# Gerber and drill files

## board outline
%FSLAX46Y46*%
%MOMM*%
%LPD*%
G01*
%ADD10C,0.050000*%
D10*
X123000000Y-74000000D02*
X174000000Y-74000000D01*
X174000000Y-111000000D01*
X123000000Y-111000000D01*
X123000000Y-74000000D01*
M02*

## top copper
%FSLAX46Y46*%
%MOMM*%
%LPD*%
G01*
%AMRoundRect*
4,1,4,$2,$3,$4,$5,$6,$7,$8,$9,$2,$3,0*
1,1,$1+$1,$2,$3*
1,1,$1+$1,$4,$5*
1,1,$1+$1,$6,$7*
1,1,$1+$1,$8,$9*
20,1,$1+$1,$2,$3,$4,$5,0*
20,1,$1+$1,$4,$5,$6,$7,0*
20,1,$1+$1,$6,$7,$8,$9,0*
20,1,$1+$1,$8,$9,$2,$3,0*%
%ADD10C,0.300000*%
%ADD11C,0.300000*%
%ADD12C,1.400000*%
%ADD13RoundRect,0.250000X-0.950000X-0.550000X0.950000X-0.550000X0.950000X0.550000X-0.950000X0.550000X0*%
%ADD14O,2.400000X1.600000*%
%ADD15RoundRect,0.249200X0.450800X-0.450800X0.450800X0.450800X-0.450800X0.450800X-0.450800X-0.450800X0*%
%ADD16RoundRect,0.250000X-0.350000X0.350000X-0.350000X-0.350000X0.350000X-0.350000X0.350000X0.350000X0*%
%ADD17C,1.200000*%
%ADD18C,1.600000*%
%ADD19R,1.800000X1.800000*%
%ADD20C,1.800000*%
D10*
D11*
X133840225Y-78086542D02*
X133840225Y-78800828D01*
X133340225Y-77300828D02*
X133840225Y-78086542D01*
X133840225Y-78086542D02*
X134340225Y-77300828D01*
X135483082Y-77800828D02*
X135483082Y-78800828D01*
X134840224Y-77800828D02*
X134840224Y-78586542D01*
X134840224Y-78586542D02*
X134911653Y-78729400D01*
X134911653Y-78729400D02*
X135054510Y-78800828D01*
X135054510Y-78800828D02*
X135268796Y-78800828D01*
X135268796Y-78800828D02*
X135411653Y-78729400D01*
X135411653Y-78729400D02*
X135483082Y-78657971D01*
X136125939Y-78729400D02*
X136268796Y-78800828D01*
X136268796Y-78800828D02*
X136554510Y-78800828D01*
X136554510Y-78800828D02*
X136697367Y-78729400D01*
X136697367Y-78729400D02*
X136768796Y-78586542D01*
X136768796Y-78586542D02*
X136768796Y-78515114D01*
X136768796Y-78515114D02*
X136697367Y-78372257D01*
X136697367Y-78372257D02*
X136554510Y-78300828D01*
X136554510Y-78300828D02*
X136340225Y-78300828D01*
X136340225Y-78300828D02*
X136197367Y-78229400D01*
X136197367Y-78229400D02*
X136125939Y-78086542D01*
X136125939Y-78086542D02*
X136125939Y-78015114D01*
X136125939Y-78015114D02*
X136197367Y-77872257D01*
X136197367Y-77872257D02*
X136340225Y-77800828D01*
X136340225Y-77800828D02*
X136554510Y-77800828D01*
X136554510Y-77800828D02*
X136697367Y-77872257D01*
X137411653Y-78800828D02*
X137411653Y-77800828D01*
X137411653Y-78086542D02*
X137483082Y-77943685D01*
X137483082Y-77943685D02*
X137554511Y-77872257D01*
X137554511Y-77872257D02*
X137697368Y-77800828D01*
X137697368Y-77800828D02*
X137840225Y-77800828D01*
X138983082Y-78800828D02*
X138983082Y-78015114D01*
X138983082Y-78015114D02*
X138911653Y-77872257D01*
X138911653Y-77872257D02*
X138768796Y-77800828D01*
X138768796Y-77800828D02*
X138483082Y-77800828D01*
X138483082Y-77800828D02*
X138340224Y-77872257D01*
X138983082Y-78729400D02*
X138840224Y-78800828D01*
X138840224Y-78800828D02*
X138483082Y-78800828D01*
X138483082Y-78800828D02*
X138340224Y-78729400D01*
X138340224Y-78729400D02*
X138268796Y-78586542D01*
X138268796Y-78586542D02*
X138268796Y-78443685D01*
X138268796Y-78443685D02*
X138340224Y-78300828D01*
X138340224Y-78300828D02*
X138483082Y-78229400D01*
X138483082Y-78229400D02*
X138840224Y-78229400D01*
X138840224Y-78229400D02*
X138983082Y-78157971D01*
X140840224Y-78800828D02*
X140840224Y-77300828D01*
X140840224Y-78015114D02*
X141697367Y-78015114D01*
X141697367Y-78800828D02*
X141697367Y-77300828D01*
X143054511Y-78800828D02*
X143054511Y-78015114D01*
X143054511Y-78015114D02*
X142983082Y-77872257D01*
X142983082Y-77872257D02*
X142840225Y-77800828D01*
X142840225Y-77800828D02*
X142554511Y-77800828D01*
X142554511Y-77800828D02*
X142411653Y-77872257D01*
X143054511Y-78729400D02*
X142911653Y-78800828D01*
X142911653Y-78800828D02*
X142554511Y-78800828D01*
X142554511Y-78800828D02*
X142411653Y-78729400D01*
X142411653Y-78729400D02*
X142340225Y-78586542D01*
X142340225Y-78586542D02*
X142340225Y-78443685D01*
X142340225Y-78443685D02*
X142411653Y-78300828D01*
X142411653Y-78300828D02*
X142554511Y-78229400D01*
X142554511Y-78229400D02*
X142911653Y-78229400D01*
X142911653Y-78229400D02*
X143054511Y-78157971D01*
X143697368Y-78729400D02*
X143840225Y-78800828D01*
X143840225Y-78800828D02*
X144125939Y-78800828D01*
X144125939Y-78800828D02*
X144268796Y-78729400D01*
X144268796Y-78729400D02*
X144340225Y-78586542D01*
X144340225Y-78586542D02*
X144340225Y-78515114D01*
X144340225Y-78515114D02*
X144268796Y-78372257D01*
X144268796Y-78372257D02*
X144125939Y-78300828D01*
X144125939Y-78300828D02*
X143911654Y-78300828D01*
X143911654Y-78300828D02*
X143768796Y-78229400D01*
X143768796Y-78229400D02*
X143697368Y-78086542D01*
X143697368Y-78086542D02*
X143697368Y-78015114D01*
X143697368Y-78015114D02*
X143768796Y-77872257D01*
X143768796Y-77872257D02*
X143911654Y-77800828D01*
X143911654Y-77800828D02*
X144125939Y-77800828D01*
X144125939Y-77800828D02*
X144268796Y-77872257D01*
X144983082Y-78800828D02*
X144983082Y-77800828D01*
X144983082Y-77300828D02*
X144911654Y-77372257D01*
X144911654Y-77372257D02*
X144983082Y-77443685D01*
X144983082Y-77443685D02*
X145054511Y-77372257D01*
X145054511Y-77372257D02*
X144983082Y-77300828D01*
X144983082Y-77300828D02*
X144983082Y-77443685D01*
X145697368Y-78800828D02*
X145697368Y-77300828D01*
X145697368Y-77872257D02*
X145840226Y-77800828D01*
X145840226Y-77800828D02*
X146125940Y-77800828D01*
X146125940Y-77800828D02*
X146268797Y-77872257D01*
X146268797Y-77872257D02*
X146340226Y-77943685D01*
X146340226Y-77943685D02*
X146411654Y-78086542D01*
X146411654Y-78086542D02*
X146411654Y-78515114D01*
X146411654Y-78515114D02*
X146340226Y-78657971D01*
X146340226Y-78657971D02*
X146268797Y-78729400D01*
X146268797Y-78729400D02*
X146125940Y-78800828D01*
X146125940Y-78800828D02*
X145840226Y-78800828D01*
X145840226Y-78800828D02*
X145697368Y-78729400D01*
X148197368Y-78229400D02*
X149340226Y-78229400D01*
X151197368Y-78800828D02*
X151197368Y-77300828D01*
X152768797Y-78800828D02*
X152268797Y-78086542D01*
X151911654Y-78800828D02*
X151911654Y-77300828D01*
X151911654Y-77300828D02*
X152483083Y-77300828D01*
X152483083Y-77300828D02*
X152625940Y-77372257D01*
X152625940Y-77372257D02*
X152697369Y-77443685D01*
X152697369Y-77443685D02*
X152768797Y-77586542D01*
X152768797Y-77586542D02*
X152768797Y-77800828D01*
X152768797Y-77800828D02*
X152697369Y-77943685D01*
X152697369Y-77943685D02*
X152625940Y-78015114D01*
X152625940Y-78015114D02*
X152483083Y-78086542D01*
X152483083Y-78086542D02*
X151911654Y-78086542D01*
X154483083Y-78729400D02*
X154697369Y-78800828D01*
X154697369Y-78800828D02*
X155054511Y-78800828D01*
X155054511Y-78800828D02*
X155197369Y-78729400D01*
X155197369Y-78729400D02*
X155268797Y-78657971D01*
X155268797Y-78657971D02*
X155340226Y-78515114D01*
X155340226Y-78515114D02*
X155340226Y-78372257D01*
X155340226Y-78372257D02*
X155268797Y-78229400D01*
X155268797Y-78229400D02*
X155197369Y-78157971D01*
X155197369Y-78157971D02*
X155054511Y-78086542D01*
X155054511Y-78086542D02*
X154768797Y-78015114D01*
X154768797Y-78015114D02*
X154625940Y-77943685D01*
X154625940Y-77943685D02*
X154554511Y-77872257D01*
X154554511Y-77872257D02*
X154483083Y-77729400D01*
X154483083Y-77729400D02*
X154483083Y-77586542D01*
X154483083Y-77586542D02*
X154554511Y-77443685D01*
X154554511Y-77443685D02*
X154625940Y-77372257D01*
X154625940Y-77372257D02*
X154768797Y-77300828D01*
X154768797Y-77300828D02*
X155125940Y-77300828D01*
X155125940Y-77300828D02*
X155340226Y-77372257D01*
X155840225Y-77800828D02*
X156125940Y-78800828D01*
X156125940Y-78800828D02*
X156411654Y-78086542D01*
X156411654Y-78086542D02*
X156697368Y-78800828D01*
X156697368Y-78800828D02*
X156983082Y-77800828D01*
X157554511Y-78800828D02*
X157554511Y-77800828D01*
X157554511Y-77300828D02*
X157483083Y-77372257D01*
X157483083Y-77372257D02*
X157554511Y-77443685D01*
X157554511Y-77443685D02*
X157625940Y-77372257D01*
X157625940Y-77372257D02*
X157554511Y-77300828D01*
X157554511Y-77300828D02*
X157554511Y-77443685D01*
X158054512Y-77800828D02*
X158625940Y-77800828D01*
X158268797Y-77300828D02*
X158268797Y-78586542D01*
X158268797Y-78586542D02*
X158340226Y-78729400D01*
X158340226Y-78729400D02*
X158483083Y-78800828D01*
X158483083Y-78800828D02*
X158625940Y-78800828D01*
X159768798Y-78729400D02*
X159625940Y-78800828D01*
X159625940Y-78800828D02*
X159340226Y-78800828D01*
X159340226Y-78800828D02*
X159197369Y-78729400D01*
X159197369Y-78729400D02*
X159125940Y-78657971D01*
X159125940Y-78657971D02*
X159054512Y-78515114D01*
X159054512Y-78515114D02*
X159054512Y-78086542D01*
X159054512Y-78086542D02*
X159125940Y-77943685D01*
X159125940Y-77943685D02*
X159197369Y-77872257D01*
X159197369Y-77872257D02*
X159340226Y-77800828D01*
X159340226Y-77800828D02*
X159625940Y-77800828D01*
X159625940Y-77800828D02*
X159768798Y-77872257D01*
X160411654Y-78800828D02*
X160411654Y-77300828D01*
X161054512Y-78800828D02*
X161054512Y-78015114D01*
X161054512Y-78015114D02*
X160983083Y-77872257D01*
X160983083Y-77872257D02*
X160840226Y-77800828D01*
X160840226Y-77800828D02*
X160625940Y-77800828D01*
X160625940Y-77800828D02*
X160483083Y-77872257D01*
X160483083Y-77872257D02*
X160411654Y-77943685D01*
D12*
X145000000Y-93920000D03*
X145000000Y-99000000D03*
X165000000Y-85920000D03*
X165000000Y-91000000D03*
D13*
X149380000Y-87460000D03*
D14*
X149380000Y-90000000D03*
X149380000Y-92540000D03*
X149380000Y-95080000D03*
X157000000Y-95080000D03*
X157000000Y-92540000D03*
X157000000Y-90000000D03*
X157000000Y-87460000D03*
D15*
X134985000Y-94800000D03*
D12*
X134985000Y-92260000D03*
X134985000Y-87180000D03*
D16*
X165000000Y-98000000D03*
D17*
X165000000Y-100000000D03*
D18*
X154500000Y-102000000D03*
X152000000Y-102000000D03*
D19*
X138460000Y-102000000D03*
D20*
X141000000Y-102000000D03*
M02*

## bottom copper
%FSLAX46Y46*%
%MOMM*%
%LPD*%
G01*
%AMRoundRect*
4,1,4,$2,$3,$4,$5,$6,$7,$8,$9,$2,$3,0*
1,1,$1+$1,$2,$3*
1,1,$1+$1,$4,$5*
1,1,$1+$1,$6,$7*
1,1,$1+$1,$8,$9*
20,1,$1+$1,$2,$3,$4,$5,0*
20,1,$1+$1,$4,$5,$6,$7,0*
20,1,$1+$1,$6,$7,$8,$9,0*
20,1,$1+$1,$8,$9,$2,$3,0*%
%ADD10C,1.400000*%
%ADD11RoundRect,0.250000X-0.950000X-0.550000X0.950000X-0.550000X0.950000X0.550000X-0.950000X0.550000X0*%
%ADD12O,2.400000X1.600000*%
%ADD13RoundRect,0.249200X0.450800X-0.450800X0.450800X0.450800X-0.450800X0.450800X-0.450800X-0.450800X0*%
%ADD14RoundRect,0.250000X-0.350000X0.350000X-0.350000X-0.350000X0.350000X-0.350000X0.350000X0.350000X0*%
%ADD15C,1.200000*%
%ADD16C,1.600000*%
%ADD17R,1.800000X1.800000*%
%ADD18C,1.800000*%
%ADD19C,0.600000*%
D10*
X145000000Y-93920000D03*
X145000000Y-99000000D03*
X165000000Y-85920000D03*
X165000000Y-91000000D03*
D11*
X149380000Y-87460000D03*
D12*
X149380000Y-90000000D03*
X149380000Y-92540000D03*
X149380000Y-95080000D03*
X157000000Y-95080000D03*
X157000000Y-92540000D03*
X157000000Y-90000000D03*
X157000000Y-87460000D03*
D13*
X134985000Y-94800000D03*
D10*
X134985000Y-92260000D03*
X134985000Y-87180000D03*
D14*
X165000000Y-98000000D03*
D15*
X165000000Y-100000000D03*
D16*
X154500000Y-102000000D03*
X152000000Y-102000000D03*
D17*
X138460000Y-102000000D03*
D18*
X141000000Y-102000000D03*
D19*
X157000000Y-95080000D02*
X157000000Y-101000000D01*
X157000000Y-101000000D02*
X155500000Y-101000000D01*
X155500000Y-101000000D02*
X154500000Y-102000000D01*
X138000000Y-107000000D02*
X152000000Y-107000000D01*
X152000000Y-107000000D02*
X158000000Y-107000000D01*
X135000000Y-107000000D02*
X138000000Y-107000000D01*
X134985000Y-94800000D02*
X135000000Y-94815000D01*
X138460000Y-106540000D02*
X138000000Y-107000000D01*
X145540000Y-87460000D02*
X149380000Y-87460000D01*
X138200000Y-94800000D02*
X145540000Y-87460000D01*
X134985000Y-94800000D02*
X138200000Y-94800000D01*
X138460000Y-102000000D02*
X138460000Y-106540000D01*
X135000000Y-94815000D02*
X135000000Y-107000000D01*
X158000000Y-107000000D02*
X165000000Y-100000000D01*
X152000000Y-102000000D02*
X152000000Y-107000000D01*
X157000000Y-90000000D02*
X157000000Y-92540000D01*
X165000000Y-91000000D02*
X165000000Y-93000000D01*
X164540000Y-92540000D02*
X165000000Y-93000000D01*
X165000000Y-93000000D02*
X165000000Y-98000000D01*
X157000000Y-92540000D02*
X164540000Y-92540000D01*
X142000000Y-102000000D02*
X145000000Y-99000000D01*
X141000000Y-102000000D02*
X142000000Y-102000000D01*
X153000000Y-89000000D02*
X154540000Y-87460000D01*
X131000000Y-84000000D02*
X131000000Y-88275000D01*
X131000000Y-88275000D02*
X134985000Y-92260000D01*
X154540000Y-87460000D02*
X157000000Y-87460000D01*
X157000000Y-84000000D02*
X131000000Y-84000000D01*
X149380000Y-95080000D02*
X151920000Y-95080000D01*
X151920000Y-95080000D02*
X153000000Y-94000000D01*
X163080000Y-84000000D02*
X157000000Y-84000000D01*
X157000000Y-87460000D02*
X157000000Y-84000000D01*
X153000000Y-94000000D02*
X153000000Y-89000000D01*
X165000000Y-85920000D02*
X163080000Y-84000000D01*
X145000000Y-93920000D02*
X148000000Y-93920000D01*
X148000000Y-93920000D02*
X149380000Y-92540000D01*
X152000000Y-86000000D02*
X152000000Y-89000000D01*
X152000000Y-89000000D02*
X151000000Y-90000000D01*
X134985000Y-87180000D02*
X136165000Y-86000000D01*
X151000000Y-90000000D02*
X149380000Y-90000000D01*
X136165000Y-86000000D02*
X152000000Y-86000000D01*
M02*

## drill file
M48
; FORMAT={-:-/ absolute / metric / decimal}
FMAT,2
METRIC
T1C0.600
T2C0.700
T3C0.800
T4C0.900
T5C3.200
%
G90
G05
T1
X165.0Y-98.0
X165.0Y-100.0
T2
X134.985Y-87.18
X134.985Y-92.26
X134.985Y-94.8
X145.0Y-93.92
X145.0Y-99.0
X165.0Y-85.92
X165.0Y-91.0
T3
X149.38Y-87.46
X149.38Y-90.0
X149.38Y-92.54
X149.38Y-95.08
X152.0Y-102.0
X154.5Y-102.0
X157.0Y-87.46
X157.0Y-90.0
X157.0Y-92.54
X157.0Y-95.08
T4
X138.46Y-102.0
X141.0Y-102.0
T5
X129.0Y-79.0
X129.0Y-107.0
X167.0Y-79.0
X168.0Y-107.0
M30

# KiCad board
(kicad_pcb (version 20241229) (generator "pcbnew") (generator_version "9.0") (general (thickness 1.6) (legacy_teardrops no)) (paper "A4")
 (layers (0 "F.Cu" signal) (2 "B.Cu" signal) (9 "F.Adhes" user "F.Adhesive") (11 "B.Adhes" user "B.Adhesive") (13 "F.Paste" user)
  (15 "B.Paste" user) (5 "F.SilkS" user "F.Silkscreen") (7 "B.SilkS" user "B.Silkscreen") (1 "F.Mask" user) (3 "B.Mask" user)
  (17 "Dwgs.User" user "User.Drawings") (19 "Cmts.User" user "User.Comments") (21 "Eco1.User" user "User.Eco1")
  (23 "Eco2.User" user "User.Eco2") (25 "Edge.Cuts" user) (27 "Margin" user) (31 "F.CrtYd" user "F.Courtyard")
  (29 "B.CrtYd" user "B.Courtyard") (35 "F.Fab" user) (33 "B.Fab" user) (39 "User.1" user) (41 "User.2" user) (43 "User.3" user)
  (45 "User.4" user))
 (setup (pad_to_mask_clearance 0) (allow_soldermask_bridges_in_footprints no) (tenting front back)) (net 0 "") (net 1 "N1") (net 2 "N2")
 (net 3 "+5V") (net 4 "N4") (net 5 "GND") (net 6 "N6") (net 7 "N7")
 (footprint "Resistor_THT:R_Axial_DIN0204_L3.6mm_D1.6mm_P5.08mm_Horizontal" (layer "F.Cu") (at 145 93.92 -90)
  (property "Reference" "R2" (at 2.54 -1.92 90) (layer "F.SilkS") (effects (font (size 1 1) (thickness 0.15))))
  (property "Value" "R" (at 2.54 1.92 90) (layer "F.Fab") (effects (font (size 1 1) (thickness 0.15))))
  (pad "1" thru_hole circle (at 0 0 270) (size 1.4 1.4) (drill 0.7) (layers "*.Cu" "*.Mask") (remove_unused_layers no) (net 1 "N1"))
  (pad "2" thru_hole circle (at 5.08 0 270) (size 1.4 1.4) (drill 0.7) (layers "*.Cu" "*.Mask") (remove_unused_layers no) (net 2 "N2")))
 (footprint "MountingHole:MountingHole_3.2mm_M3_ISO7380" (layer "F.Cu") (at 168 107)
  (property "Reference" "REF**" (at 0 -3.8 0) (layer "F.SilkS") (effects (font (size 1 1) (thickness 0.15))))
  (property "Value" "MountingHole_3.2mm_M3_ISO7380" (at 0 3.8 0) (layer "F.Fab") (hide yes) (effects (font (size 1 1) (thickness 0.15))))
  (pad "" np_thru_hole circle (at 0 0) (size 3.2 3.2) (drill 3.2) (layers "*.Cu" "*.Mask")))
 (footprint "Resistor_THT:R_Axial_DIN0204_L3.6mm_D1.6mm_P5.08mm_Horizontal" (layer "F.Cu") (at 165 85.92 -90)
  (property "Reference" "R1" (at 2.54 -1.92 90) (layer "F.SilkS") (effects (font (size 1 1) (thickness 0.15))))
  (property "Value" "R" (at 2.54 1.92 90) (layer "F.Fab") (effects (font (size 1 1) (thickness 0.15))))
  (pad "1" thru_hole circle (at 0 0 270) (size 1.4 1.4) (drill 0.7) (layers "*.Cu" "*.Mask") (remove_unused_layers no) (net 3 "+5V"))
  (pad "2" thru_hole circle (at 5.08 0 270) (size 1.4 1.4) (drill 0.7) (layers "*.Cu" "*.Mask") (remove_unused_layers no) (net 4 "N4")))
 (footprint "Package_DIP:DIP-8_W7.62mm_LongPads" (layer "F.Cu") (at 149.38 87.46)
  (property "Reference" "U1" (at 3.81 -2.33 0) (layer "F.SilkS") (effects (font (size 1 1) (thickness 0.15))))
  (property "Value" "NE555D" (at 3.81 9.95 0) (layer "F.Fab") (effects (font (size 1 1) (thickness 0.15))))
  (pad "1" thru_hole roundrect (at 0 0) (size 2.4 1.6) (drill 0.8) (layers "*.Cu" "*.Mask") (remove_unused_layers no)
   (roundrect_rratio 0.15625) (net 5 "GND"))
  (pad "2" thru_hole oval (at 0 2.54) (size 2.4 1.6) (drill 0.8) (layers "*.Cu" "*.Mask") (remove_unused_layers no) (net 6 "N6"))
  (pad "3" thru_hole oval (at 0 5.08) (size 2.4 1.6) (drill 0.8) (layers "*.Cu" "*.Mask") (remove_unused_layers no) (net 1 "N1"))
  (pad "4" thru_hole oval (at 0 7.62) (size 2.4 1.6) (drill 0.8) (layers "*.Cu" "*.Mask") (remove_unused_layers no) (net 3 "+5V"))
  (pad "5" thru_hole oval (at 7.62 7.62) (size 2.4 1.6) (drill 0.8) (layers "*.Cu" "*.Mask") (remove_unused_layers no) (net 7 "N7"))
  (pad "6" thru_hole oval (at 7.62 5.08) (size 2.4 1.6) (drill 0.8) (layers "*.Cu" "*.Mask") (remove_unused_layers no) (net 4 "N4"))
  (pad "7" thru_hole oval (at 7.62 2.54) (size 2.4 1.6) (drill 0.8) (layers "*.Cu" "*.Mask") (remove_unused_layers no) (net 4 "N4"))
  (pad "8" thru_hole oval (at 7.62 0) (size 2.4 1.6) (drill 0.8) (layers "*.Cu" "*.Mask") (remove_unused_layers no) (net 3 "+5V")))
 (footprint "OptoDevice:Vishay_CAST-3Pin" (layer "F.Cu") (at 134.985 94.8 90)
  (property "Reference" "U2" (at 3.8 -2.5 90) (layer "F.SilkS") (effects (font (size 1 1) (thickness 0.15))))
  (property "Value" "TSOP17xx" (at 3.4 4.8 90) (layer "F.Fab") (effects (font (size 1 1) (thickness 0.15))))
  (pad "1" thru_hole roundrect (at 0 0 90) (size 1.4 1.4) (drill 0.7) (layers "*.Cu" "*.Mask") (remove_unused_layers no)
   (roundrect_rratio 0.178) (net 5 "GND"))
  (pad "2" thru_hole circle (at 2.54 0 90) (size 1.4 1.4) (drill 0.7) (layers "*.Cu" "*.Mask") (remove_unused_layers no) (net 3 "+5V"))
  (pad "3" thru_hole circle (at 7.62 0 90) (size 1.4 1.4) (drill 0.7) (layers "*.Cu" "*.Mask") (remove_unused_layers no) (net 6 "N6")))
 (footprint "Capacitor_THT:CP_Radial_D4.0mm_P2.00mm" (layer "F.Cu") (at 165 98 -90)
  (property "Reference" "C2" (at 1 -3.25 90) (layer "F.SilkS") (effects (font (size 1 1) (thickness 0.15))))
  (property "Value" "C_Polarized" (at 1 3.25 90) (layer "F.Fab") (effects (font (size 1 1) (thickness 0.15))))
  (pad "1" thru_hole roundrect (at 0 0 270) (size 1.2 1.2) (drill 0.6) (layers "*.Cu" "*.Mask") (remove_unused_layers no)
   (roundrect_rratio 0.208333) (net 4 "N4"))
  (pad "2" thru_hole circle (at 2 0 270) (size 1.2 1.2) (drill 0.6) (layers "*.Cu" "*.Mask") (remove_unused_layers no) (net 5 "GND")))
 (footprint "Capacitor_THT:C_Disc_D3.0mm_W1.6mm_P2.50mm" (layer "F.Cu") (at 154.5 102 180)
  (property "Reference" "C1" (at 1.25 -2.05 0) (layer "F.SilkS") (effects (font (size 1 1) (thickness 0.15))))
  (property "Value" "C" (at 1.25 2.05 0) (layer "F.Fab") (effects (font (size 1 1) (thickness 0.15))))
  (pad "1" thru_hole circle (at 0 0 180) (size 1.6 1.6) (drill 0.8) (layers "*.Cu" "*.Mask") (remove_unused_layers no) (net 7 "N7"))
  (pad "2" thru_hole circle (at 2.5 0 180) (size 1.6 1.6) (drill 0.8) (layers "*.Cu" "*.Mask") (remove_unused_layers no) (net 5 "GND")))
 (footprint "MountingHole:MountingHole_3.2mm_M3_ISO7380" (layer "F.Cu") (at 167 79)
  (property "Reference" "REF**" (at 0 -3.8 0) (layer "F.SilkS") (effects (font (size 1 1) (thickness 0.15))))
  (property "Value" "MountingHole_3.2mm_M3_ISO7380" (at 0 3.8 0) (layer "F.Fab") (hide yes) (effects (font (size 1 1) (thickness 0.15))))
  (pad "" np_thru_hole circle (at 0 0) (size 3.2 3.2) (drill 3.2) (layers "*.Cu" "*.Mask")))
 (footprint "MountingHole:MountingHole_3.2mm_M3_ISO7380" (layer "F.Cu") (at 129 107)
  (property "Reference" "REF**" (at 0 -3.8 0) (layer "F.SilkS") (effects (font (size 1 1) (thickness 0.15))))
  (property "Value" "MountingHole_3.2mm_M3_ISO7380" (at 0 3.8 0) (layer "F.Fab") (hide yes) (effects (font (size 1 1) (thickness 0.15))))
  (pad "" np_thru_hole circle (at 0 0) (size 3.2 3.2) (drill 3.2) (layers "*.Cu" "*.Mask")))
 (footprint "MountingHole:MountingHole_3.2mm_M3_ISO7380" (layer "F.Cu") (at 129 79)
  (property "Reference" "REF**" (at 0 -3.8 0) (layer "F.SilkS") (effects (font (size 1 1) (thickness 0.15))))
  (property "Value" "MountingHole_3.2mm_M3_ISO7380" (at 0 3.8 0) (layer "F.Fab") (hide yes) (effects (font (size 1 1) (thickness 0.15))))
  (pad "" np_thru_hole circle (at 0 0) (size 3.2 3.2) (drill 3.2) (layers "*.Cu" "*.Mask")))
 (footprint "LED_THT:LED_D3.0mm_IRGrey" (layer "F.Cu") (at 138.46 102)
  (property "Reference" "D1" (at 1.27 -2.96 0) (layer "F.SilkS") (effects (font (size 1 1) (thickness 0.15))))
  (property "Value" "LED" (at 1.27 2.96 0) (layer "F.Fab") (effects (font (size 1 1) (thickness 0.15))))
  (pad "1" thru_hole rect (at 0 0) (size 1.8 1.8) (drill 0.9) (layers "*.Cu" "*.Mask") (remove_unused_layers no) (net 5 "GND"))
  (pad "2" thru_hole circle (at 2.54 0) (size 1.8 1.8) (drill 0.9) (layers "*.Cu" "*.Mask") (remove_unused_layers no) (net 2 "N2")))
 (gr_poly (pts (xy 123 74) (xy 174 74) (xy 174 111) (xy 123 111)) (stroke (width 0.05) (type solid)) (fill no) (layer "Edge.Cuts"))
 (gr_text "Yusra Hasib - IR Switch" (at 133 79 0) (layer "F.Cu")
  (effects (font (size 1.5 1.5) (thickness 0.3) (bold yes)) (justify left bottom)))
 (segment (start 157 95.08) (end 157 101) (width 0.6) (layer "B.Cu") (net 7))
 (segment (start 157 101) (end 155.5 101) (width 0.6) (layer "B.Cu") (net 7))
 (segment (start 155.5 101) (end 154.5 102) (width 0.6) (layer "B.Cu") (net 7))
 (segment (start 138 107) (end 152 107) (width 0.6) (layer "B.Cu") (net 5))
 (segment (start 152 107) (end 158 107) (width 0.6) (layer "B.Cu") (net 5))
 (segment (start 135 107) (end 138 107) (width 0.6) (layer "B.Cu") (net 5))
 (segment (start 134.985 94.8) (end 135 94.815) (width 0.6) (layer "B.Cu") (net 5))
 (segment (start 138.46 106.54) (end 138 107) (width 0.6) (layer "B.Cu") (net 5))
 (segment (start 145.54 87.46) (end 149.38 87.46) (width 0.6) (layer "B.Cu") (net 5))
 (segment (start 138.2 94.8) (end 145.54 87.46) (width 0.6) (layer "B.Cu") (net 5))
 (segment (start 134.985 94.8) (end 138.2 94.8) (width 0.6) (layer "B.Cu") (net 5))
 (segment (start 138.46 102) (end 138.46 106.54) (width 0.6) (layer "B.Cu") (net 5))
 (segment (start 135 94.815) (end 135 107) (width 0.6) (layer "B.Cu") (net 5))
 (segment (start 158 107) (end 165 100) (width 0.6) (layer "B.Cu") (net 5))
 (segment (start 152 102) (end 152 107) (width 0.6) (layer "B.Cu") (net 5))
 (segment (start 157 90) (end 157 92.54) (width 0.6) (layer "B.Cu") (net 4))
 (segment (start 165 91) (end 165 93) (width 0.6) (layer "B.Cu") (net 4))
 (segment (start 164.54 92.54) (end 165 93) (width 0.6) (layer "B.Cu") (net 4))
 (segment (start 165 93) (end 165 98) (width 0.6) (layer "B.Cu") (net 4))
 (segment (start 157 92.54) (end 164.54 92.54) (width 0.6) (layer "B.Cu") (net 4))
 (segment (start 142 102) (end 145 99) (width 0.6) (layer "B.Cu") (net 2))
 (segment (start 141 102) (end 142 102) (width 0.6) (layer "B.Cu") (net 2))
 (segment (start 153 89) (end 154.54 87.46) (width 0.6) (layer "B.Cu") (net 3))
 (segment (start 131 84) (end 131 88.275) (width 0.6) (layer "B.Cu") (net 3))
 (segment (start 131 88.275) (end 134.985 92.26) (width 0.6) (layer "B.Cu") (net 3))
 (segment (start 154.54 87.46) (end 157 87.46) (width 0.6) (layer "B.Cu") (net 3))
 (segment (start 157 84) (end 131 84) (width 0.6) (layer "B.Cu") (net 3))
 (segment (start 149.38 95.08) (end 151.92 95.08) (width 0.6) (layer "B.Cu") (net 3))
 (segment (start 151.92 95.08) (end 153 94) (width 0.6) (layer "B.Cu") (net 3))
 (segment (start 163.08 84) (end 157 84) (width 0.6) (layer "B.Cu") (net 3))
 (segment (start 157 87.46) (end 157 84) (width 0.6) (layer "B.Cu") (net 3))
 (segment (start 153 94) (end 153 89) (width 0.6) (layer "B.Cu") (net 3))
 (segment (start 165 85.92) (end 163.08 84) (width 0.6) (layer "B.Cu") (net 3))
 (segment (start 145 93.92) (end 148 93.92) (width 0.6) (layer "B.Cu") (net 1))
 (segment (start 148 93.92) (end 149.38 92.54) (width 0.6) (layer "B.Cu") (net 1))
 (segment (start 152 86) (end 152 89) (width 0.6) (layer "B.Cu") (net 6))
 (segment (start 152 89) (end 151 90) (width 0.6) (layer "B.Cu") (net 6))
 (segment (start 134.985 87.18) (end 136.165 86) (width 0.6) (layer "B.Cu") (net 6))
 (segment (start 151 90) (end 149.38 90) (width 0.6) (layer "B.Cu") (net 6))
 (segment (start 136.165 86) (end 152 86) (width 0.6) (layer "B.Cu") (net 6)))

